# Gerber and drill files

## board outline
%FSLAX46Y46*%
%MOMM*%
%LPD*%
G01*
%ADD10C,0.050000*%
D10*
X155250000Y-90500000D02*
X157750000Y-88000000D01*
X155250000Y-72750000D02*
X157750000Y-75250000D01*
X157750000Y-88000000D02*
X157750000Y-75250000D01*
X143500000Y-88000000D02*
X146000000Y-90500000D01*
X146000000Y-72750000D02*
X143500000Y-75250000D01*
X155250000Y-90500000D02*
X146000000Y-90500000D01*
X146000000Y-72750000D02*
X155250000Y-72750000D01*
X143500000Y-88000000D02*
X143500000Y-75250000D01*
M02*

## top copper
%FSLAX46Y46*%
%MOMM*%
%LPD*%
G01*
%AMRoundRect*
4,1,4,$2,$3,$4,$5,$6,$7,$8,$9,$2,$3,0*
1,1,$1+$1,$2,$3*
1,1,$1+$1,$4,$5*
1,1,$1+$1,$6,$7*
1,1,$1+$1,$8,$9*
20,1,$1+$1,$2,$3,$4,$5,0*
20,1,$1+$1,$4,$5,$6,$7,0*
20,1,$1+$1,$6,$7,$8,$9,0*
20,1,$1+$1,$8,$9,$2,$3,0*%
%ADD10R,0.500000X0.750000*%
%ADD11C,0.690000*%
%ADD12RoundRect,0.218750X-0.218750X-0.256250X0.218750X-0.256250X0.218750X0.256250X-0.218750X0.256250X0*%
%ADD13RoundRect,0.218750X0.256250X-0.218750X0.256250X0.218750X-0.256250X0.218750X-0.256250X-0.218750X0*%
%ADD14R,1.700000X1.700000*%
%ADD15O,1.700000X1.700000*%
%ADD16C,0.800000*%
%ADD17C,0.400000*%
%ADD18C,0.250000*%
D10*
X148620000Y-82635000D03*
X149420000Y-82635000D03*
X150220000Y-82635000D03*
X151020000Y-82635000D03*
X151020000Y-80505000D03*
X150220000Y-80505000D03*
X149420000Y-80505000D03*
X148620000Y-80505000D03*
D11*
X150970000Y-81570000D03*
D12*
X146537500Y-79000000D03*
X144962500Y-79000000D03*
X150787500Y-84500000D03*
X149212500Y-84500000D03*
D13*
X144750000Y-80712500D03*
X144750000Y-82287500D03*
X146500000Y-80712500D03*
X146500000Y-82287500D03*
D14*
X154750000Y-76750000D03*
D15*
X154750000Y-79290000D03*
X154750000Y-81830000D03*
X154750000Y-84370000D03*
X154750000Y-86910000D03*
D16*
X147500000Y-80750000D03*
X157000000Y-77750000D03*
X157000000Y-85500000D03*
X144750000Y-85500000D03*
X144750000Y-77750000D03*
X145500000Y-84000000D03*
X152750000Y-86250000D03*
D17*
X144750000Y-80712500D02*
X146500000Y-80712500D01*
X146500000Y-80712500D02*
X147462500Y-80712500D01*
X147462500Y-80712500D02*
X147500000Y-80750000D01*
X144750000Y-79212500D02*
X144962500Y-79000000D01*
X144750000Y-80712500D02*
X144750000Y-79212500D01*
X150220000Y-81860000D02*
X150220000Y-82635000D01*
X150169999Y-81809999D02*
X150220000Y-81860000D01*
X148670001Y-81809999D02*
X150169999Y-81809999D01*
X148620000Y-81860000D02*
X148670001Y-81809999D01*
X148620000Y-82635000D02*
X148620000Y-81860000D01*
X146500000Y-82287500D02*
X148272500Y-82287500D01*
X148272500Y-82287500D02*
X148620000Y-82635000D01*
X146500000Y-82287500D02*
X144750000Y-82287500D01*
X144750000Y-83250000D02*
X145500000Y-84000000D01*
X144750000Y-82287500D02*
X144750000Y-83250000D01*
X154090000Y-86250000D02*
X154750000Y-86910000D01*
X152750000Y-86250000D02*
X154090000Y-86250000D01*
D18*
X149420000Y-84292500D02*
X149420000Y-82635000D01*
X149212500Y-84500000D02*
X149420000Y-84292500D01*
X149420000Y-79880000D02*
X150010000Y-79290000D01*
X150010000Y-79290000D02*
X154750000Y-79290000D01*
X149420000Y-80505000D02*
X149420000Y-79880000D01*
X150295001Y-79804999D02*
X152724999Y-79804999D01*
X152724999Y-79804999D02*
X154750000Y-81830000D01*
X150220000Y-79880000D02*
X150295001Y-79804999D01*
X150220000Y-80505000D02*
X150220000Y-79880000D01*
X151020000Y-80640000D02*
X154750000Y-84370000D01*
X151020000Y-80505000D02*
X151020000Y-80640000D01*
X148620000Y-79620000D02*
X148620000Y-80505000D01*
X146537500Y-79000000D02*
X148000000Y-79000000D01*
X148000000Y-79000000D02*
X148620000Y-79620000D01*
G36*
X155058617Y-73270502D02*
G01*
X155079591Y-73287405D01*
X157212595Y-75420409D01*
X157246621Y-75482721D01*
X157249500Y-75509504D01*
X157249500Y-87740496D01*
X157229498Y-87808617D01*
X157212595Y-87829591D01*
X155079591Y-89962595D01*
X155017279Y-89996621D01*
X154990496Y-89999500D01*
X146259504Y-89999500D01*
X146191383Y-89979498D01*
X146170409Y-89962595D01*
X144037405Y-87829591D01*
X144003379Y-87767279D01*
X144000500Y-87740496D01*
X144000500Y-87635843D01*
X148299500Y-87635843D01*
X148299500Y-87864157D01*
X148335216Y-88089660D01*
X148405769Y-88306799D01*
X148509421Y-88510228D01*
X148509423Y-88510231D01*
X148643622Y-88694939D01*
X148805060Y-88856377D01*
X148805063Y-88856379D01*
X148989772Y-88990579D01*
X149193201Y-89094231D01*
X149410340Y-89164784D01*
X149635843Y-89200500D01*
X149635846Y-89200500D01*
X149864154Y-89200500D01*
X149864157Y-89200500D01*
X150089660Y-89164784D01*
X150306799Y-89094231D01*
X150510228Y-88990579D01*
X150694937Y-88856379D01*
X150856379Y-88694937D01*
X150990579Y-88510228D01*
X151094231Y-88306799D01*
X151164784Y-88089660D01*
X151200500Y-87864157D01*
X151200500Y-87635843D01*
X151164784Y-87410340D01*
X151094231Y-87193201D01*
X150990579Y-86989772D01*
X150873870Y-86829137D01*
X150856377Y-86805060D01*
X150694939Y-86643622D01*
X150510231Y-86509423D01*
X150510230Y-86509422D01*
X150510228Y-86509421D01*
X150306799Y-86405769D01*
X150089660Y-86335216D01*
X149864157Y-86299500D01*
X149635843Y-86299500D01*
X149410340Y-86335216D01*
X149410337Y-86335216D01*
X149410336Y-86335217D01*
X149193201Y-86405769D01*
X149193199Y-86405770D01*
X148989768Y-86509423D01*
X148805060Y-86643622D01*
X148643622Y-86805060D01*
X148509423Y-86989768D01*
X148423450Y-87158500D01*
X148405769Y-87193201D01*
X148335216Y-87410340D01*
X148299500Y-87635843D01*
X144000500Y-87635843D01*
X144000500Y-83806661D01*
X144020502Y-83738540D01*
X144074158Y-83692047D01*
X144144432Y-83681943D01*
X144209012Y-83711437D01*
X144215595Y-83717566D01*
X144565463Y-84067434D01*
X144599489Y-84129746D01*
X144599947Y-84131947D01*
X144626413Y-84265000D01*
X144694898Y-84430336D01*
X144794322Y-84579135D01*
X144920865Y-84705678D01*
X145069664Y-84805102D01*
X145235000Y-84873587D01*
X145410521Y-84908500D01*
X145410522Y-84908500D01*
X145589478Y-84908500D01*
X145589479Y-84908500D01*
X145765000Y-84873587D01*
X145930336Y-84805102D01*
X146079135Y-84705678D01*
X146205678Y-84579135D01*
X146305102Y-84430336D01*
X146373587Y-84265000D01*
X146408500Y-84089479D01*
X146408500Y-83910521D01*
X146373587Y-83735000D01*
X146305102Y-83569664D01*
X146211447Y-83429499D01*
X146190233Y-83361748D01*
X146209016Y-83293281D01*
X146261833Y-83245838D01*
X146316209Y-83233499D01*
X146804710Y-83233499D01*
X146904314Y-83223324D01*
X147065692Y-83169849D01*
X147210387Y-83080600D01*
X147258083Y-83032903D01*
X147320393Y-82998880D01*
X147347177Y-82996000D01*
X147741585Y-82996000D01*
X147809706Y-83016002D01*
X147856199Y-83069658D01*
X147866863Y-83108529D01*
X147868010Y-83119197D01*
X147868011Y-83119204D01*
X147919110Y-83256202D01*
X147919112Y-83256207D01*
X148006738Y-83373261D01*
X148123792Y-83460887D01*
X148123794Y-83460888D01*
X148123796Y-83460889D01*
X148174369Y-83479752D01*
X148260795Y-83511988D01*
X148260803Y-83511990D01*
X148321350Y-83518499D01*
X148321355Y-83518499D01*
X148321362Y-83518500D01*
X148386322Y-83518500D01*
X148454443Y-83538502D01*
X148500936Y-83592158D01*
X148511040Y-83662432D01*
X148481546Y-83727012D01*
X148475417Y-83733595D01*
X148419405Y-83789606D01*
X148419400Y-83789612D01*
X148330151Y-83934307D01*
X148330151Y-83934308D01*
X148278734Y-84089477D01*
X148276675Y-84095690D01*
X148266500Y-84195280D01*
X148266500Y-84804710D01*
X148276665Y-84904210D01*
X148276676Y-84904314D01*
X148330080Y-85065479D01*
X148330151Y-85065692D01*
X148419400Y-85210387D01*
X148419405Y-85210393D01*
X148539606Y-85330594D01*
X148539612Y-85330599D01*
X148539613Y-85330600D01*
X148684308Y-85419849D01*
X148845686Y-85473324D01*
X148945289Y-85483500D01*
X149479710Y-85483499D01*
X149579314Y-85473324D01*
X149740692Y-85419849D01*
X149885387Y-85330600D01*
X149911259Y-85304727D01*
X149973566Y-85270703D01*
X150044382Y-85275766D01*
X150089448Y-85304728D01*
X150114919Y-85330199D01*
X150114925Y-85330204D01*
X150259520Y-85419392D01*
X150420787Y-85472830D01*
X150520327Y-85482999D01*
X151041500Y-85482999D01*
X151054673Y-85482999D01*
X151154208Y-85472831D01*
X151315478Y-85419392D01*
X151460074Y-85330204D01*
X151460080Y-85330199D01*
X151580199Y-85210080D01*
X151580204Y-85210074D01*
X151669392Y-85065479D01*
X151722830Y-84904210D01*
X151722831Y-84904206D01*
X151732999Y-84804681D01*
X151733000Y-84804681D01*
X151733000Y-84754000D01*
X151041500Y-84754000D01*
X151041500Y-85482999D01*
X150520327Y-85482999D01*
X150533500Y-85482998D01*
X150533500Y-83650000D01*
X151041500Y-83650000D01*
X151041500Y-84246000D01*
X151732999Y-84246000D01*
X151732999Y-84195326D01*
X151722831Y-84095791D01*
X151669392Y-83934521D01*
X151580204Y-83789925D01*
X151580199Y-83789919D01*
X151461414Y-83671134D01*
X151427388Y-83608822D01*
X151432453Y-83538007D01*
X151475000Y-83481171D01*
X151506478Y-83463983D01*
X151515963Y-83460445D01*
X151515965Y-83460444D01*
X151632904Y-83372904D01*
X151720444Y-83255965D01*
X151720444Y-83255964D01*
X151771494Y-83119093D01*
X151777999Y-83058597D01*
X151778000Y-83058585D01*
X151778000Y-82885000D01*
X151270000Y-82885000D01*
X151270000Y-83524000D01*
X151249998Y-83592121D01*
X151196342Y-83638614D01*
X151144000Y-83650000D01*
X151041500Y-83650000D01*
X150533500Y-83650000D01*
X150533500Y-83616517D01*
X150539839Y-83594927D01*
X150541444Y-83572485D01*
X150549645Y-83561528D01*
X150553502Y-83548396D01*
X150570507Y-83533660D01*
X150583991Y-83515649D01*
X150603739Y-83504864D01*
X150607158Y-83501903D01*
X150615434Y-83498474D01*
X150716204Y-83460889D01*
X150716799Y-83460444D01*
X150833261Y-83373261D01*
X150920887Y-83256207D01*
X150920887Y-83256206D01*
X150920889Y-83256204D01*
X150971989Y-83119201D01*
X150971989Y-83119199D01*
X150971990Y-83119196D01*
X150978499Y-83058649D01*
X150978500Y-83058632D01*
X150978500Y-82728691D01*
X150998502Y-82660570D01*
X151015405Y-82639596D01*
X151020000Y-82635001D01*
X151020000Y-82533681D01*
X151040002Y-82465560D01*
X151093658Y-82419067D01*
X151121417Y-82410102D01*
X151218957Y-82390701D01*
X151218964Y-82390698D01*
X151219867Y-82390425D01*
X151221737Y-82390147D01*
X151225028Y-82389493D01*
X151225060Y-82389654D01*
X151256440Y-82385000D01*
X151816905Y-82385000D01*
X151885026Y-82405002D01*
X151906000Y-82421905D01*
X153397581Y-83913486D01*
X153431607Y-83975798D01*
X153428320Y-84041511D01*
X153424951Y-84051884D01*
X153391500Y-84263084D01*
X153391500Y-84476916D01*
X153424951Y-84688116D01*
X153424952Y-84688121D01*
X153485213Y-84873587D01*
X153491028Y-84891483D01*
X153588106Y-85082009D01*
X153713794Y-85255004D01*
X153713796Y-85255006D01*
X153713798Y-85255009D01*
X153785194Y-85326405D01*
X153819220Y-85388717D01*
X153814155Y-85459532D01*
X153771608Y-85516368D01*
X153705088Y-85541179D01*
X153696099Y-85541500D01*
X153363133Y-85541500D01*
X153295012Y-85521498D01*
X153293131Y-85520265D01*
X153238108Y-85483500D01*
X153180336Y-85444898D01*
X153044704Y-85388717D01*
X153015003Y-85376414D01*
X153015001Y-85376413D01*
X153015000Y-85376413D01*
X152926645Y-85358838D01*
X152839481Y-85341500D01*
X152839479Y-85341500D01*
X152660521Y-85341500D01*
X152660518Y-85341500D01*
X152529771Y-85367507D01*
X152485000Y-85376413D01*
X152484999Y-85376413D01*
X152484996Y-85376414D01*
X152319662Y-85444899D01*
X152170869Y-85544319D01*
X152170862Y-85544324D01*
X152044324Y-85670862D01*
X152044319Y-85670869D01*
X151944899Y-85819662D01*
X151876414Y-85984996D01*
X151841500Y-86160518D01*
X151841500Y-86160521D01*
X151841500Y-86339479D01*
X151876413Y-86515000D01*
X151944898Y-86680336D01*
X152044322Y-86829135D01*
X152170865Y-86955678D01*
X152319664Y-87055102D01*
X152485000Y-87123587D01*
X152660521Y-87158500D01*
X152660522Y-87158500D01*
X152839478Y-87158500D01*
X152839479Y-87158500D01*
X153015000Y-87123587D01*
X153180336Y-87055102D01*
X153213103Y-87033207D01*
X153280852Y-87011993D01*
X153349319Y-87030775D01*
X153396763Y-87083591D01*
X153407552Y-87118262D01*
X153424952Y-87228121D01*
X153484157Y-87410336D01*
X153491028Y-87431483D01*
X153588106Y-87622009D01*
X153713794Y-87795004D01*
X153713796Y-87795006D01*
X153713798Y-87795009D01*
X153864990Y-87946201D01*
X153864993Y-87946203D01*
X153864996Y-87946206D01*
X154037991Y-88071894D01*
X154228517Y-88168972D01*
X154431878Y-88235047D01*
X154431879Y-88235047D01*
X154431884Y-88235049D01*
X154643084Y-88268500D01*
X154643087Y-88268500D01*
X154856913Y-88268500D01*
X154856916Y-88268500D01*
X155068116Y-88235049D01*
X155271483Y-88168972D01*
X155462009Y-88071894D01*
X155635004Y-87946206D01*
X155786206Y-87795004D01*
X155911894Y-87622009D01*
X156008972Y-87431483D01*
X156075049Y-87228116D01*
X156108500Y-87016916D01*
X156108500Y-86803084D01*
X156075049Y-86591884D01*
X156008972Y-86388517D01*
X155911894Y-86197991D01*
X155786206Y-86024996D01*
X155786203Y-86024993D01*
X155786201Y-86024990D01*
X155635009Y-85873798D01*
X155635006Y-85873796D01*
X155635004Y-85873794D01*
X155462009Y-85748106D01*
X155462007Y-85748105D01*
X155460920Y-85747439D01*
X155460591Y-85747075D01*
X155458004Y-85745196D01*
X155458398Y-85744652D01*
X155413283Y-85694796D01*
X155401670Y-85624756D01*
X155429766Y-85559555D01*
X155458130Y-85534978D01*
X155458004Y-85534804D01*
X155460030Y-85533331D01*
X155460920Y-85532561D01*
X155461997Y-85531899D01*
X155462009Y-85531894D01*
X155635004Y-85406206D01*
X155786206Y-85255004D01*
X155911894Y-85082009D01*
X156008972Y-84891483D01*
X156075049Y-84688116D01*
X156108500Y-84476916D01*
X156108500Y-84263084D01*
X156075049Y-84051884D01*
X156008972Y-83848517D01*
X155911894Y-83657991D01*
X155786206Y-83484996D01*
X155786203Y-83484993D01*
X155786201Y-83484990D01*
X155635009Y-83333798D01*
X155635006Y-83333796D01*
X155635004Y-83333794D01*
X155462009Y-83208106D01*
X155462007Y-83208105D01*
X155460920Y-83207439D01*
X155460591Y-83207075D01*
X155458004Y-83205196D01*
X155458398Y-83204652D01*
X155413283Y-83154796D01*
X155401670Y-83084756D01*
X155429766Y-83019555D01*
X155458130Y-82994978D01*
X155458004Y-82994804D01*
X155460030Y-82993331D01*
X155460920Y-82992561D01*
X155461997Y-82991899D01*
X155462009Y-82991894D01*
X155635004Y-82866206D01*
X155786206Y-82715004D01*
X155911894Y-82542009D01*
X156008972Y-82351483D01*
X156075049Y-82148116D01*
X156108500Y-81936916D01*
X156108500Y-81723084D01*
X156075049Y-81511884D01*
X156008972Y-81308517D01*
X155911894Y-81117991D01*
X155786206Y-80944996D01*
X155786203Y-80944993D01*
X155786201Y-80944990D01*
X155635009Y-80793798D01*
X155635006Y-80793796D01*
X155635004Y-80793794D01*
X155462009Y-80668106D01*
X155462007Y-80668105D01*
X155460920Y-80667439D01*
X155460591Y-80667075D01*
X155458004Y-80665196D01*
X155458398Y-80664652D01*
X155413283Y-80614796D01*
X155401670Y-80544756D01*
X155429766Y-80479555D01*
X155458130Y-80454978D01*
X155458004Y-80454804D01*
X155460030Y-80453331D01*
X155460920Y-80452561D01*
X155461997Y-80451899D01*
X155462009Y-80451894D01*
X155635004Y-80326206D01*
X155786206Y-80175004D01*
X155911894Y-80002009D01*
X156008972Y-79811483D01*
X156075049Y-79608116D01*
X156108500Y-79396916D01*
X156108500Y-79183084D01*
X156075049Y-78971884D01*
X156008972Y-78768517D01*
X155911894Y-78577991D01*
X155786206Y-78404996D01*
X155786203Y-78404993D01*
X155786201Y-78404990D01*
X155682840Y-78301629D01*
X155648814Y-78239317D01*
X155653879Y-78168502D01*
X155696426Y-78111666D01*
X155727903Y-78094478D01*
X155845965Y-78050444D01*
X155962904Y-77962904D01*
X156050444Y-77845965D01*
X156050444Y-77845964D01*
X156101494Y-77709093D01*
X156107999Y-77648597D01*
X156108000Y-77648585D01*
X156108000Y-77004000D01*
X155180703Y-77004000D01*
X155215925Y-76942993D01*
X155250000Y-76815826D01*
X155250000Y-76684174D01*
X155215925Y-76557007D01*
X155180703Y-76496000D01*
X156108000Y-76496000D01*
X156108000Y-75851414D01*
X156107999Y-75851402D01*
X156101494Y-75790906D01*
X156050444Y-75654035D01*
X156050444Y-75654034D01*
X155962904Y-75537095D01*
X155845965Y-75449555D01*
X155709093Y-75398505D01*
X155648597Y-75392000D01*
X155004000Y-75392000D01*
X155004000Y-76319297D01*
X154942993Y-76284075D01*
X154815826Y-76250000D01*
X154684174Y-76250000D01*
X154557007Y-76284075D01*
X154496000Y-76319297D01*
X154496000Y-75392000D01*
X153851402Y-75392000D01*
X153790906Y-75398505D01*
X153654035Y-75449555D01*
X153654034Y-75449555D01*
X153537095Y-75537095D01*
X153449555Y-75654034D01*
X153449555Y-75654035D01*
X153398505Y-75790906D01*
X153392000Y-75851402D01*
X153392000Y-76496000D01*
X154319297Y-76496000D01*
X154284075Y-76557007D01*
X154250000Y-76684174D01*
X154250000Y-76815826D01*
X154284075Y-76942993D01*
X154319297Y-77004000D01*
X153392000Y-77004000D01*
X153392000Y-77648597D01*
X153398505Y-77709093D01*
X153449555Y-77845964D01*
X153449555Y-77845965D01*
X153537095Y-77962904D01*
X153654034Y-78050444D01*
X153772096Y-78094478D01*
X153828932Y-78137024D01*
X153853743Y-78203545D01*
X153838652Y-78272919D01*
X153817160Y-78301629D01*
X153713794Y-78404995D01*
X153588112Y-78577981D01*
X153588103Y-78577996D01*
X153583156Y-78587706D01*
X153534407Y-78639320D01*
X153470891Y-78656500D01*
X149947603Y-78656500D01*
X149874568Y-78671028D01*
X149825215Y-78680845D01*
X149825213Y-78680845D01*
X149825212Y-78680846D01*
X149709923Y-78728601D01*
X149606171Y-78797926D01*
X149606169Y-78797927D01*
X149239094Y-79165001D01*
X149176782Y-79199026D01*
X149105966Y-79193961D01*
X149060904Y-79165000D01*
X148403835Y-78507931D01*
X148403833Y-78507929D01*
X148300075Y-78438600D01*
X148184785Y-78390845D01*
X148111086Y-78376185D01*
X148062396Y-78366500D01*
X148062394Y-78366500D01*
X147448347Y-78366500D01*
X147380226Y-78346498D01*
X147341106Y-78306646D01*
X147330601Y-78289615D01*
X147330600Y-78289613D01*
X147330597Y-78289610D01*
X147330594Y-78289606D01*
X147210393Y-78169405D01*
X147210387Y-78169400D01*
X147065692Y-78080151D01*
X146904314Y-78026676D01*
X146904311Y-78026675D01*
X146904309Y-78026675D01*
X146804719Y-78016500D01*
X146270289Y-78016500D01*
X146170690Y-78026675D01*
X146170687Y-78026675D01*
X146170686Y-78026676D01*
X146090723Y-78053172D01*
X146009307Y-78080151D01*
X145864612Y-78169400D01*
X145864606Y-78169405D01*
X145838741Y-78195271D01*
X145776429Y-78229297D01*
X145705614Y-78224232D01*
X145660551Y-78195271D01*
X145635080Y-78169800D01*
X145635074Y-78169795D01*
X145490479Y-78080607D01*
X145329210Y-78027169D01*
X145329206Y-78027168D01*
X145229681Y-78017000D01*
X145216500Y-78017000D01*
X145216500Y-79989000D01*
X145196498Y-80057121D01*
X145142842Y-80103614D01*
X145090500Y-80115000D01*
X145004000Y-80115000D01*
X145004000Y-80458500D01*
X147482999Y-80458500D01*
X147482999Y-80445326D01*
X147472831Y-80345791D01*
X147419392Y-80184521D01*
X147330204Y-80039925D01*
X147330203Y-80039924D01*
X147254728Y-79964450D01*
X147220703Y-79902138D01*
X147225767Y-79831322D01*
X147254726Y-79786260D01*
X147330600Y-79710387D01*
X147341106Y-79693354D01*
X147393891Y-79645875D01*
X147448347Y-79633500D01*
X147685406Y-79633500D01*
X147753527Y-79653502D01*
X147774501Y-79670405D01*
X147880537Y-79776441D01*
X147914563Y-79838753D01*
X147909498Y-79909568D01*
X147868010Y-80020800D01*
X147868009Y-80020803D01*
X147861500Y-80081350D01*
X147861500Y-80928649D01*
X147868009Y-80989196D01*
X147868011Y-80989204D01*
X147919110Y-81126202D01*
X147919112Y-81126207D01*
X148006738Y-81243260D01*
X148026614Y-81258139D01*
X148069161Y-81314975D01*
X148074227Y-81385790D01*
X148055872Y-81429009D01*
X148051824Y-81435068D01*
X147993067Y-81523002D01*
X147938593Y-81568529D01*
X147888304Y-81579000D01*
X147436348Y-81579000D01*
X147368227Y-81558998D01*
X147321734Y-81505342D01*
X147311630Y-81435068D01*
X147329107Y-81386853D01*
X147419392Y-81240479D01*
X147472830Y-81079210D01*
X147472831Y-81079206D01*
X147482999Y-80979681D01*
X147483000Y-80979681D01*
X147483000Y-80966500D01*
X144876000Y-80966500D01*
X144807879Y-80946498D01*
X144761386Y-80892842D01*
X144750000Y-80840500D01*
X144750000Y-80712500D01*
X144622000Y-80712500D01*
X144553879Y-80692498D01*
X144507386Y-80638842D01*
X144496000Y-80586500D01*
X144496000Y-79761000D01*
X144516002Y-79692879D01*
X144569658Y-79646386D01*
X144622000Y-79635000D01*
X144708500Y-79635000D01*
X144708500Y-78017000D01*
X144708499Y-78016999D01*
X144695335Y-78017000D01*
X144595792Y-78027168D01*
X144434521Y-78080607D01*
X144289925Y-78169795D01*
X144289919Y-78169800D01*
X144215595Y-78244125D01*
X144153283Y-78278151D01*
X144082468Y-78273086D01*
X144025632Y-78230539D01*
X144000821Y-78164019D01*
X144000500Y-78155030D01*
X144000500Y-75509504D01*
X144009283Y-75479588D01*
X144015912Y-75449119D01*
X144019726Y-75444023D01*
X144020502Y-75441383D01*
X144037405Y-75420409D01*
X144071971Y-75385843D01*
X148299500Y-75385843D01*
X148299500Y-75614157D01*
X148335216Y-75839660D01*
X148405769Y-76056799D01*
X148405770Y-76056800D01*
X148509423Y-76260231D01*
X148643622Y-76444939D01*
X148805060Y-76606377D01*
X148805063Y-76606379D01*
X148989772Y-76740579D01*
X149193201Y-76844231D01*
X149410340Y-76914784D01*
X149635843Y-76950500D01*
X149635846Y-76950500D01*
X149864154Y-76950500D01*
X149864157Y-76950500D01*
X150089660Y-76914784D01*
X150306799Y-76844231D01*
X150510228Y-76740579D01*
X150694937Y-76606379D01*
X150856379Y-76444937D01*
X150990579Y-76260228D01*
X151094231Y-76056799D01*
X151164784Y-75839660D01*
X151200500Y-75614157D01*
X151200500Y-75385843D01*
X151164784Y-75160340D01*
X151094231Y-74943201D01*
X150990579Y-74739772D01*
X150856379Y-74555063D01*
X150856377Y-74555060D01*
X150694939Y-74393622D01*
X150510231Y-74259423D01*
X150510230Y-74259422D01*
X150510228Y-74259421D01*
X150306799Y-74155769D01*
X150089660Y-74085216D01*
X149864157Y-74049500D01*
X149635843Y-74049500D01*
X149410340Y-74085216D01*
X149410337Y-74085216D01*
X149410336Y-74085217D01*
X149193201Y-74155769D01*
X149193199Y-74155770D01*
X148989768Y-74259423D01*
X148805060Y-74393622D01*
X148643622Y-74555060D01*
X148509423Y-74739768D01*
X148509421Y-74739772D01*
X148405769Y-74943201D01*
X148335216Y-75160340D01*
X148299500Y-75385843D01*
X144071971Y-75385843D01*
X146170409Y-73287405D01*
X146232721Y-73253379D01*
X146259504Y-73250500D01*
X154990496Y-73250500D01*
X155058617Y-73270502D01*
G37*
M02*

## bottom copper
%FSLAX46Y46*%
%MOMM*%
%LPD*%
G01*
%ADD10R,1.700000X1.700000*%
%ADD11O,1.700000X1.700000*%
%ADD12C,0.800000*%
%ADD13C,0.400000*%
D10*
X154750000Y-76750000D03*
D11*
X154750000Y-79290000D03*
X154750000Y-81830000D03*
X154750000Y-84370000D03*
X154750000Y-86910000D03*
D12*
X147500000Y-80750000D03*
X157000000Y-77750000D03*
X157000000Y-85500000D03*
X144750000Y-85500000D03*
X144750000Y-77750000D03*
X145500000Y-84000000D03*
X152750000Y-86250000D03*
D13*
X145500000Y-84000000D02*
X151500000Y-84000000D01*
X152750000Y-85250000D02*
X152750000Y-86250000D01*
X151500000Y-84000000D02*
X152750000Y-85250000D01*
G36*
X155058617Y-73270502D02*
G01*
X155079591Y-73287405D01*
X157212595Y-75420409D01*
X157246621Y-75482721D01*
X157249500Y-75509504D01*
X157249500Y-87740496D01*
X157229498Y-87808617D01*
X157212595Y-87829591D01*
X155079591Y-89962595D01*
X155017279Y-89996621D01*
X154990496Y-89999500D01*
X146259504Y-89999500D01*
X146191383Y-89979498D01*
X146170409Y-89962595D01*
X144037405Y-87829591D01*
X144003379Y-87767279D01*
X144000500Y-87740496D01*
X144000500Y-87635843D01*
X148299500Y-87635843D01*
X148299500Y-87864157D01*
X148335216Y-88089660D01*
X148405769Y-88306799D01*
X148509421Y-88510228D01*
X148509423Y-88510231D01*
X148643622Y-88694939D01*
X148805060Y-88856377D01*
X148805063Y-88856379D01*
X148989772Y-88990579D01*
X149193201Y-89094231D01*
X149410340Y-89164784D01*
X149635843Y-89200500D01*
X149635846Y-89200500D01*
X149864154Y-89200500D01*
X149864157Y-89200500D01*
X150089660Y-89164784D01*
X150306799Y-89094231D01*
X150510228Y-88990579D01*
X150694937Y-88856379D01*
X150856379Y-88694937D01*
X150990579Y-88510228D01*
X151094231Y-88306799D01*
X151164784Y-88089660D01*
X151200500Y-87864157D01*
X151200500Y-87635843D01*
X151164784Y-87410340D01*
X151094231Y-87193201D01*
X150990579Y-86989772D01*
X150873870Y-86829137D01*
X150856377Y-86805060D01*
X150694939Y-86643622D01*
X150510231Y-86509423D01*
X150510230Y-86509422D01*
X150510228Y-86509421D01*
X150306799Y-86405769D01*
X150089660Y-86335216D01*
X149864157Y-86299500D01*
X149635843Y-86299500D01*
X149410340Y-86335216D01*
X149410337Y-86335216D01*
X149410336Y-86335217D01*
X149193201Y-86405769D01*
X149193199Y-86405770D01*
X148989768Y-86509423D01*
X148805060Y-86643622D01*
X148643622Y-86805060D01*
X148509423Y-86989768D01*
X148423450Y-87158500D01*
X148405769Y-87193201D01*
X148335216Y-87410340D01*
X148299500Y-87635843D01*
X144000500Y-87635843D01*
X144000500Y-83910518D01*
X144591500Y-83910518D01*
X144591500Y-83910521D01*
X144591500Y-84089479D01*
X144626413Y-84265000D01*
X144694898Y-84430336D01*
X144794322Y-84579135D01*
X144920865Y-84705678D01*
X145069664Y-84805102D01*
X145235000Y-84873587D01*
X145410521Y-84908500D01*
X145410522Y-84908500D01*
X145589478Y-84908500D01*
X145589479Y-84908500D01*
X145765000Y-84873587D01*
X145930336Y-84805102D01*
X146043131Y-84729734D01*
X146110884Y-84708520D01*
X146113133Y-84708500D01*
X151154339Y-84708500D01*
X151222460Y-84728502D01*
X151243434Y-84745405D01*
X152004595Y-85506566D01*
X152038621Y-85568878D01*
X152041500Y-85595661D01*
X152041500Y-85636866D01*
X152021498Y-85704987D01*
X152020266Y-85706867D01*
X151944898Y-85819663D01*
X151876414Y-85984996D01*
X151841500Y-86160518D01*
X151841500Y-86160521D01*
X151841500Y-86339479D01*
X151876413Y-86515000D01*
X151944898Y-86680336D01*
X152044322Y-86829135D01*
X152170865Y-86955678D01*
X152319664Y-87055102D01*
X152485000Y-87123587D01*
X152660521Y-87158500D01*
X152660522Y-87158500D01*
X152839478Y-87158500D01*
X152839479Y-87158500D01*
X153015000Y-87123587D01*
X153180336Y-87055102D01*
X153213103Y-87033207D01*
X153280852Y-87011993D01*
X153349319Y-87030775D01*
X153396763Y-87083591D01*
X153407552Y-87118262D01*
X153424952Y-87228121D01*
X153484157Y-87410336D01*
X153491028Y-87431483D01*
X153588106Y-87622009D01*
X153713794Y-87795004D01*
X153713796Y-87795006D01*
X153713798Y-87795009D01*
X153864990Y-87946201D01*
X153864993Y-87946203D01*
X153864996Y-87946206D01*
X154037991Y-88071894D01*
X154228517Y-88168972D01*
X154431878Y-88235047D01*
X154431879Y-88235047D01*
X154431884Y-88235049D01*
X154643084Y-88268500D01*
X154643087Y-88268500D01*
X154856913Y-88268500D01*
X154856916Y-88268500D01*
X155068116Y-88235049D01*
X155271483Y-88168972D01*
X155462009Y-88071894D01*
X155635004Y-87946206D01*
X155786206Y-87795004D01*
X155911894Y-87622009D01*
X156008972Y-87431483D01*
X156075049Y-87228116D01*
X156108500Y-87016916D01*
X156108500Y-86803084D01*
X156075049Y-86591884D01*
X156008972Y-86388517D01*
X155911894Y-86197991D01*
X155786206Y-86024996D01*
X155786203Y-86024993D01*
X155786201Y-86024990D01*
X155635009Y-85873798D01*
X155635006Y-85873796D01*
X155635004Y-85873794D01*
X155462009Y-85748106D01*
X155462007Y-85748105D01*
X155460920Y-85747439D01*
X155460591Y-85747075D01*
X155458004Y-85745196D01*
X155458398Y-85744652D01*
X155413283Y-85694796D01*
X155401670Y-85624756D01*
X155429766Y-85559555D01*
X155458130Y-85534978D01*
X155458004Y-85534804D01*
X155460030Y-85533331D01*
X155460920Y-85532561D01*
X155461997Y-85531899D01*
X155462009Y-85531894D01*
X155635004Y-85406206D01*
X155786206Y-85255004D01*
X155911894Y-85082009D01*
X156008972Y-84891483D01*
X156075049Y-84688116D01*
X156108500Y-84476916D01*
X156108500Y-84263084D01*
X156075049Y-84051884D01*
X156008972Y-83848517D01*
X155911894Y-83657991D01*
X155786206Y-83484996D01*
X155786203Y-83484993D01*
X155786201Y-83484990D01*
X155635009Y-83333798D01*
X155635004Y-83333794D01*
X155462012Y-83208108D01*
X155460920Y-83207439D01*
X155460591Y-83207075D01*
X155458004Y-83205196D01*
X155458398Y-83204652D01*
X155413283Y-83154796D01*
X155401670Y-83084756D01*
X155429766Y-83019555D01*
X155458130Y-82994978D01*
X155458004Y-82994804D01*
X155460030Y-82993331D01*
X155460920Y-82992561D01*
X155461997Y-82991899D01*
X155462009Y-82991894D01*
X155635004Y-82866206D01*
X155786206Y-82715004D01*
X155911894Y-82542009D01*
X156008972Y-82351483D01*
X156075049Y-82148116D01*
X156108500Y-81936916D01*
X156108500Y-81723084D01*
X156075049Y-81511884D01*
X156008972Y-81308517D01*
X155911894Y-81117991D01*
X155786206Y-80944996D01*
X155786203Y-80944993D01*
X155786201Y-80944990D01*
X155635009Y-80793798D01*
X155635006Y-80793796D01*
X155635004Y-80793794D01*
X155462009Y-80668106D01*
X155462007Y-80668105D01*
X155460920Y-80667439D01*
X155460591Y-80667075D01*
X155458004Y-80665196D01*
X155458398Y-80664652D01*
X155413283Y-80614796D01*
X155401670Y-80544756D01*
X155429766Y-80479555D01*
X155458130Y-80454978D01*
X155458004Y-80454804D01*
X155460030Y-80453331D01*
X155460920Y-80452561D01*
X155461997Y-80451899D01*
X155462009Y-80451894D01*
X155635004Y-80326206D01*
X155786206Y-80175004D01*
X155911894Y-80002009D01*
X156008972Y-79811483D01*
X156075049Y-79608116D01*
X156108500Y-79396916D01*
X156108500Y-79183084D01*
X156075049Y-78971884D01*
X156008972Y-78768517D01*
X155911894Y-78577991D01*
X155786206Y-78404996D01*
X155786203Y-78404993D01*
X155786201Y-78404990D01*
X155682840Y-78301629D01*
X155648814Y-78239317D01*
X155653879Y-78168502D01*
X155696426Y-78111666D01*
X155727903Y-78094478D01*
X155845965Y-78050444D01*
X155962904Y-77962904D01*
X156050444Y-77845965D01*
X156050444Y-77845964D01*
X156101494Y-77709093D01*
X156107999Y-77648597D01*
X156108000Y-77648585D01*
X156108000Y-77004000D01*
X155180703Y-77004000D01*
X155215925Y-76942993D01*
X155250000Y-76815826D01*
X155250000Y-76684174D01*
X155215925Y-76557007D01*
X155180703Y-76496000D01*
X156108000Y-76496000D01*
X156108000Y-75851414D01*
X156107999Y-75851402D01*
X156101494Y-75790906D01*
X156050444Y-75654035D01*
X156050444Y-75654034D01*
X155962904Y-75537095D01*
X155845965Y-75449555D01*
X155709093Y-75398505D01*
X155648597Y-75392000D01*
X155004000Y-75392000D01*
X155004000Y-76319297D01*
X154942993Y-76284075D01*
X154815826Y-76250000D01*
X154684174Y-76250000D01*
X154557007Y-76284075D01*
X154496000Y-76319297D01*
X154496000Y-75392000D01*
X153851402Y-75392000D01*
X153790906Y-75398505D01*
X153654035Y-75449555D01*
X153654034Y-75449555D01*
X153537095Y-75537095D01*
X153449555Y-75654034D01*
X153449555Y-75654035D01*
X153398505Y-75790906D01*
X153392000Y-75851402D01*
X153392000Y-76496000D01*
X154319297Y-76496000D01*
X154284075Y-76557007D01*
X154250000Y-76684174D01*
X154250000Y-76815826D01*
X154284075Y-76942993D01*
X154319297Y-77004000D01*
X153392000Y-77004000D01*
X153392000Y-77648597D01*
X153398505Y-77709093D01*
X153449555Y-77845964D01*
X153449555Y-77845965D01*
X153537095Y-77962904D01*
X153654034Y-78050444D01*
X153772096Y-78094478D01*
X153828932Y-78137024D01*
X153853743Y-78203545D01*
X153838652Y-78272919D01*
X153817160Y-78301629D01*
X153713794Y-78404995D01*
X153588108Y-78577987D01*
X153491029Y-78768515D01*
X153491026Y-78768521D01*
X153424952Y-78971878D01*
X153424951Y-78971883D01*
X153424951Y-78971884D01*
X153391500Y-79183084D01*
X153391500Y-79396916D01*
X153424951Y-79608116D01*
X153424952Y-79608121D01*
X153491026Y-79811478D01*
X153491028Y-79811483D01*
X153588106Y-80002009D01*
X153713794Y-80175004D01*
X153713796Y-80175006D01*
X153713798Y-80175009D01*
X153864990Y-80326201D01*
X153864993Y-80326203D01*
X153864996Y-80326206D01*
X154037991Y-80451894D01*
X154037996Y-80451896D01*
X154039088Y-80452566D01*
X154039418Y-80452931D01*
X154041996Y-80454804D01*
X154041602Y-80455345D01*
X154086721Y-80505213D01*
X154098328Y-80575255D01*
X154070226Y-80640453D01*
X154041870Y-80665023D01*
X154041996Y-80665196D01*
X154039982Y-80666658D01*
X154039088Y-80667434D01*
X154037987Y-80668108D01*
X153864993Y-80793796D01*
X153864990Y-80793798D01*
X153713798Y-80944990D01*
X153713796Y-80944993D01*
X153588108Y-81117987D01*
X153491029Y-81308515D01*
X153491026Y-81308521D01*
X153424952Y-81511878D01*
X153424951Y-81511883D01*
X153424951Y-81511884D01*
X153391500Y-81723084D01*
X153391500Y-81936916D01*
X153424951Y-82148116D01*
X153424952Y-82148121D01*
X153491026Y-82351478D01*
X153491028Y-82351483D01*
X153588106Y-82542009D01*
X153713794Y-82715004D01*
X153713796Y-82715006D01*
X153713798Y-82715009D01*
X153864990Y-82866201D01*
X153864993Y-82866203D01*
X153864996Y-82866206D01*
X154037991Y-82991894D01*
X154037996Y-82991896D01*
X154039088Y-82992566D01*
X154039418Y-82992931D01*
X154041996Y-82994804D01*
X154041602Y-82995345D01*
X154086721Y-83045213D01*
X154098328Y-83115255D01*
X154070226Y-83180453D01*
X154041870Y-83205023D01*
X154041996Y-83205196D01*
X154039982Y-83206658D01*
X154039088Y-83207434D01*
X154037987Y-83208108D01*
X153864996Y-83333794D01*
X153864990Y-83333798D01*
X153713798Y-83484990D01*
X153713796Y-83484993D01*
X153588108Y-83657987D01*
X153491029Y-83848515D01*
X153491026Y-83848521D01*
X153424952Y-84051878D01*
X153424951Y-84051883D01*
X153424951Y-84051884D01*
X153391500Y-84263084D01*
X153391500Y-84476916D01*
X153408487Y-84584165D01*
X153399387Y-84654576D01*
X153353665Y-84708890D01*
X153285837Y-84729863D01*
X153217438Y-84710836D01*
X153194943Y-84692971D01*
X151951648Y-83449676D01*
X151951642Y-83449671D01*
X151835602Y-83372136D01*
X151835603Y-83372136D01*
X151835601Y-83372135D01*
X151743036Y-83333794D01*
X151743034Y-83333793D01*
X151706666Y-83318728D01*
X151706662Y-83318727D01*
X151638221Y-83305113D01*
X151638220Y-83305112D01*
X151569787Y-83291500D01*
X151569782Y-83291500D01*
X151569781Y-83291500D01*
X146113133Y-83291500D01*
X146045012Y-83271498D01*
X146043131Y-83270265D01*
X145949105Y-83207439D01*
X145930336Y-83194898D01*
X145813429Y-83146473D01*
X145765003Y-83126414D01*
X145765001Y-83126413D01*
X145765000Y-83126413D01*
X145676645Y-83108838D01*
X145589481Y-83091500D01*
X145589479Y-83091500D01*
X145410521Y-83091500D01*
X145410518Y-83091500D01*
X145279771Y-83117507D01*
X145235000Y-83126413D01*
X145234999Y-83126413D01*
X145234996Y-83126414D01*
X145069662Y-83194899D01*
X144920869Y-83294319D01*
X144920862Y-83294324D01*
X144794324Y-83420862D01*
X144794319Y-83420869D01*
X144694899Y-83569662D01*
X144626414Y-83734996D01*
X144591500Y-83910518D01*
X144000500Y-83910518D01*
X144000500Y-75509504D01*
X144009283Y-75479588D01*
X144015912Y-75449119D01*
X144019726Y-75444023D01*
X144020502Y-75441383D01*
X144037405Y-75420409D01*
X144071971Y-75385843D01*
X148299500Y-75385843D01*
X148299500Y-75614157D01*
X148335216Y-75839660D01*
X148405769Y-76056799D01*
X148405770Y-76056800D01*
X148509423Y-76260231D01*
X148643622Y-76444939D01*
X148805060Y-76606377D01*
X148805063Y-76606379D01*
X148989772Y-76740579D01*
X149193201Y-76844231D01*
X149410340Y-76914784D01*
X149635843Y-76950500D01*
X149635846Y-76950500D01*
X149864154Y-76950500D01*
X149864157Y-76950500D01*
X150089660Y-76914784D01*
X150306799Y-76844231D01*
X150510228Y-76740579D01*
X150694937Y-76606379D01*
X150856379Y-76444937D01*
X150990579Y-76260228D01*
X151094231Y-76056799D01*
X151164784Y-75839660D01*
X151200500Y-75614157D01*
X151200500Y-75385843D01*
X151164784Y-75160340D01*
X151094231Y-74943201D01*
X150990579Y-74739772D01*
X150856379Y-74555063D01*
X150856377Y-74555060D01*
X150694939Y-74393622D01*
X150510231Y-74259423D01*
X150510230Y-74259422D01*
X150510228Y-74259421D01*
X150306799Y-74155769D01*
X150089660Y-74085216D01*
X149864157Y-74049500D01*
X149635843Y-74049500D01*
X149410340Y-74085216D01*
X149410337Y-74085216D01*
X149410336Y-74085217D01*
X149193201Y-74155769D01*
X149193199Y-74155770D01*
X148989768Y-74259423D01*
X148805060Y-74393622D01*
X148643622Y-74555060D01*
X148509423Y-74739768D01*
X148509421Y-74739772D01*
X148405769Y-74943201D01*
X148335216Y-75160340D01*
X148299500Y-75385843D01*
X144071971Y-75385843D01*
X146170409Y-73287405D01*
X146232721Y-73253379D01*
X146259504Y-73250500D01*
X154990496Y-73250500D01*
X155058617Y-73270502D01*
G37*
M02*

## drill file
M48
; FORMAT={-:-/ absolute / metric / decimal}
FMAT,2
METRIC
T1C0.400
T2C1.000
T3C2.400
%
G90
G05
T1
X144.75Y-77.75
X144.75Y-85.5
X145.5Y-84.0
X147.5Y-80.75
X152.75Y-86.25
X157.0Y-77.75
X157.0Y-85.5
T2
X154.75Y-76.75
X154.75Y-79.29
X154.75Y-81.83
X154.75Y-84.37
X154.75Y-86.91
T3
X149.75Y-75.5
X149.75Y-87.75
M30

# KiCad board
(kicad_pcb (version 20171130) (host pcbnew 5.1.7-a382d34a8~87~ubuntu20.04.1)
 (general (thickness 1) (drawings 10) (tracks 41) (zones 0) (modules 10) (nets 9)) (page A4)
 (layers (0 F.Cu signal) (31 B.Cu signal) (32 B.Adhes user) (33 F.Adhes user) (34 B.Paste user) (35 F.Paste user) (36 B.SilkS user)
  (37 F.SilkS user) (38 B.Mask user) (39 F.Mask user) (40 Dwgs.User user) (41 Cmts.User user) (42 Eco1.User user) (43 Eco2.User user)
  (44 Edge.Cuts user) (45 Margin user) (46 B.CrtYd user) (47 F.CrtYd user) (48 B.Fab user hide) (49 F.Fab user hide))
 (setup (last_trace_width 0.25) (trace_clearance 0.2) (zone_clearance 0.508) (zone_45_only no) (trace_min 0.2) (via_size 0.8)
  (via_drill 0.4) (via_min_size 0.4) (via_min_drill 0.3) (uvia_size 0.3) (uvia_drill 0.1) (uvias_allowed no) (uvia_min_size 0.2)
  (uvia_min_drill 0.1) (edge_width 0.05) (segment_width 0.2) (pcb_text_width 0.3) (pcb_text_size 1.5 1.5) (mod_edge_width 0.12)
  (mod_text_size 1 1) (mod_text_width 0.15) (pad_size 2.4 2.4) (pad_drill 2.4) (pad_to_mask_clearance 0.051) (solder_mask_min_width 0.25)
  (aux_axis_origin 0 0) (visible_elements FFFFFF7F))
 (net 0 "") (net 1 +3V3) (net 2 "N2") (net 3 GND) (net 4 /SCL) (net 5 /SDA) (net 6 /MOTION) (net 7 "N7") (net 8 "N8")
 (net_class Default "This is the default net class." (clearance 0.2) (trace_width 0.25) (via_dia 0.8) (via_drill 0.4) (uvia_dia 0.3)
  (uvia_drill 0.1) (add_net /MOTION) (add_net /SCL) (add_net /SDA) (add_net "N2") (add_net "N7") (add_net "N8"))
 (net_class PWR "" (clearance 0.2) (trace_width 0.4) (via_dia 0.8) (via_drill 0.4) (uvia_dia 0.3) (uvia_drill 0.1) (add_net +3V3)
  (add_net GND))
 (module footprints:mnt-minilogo (layer F.Cu) (at 146.5 86.75 90)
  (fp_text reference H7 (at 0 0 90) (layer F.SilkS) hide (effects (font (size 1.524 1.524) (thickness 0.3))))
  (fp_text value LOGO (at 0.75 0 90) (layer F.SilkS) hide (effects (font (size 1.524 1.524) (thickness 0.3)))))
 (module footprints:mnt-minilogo (layer B.Cu) (at 146 86 270)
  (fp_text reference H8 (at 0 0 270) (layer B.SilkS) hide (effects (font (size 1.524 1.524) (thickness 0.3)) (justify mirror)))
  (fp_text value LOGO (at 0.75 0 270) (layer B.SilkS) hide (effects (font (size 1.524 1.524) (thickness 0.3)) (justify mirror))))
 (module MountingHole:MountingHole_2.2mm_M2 (layer F.Cu) (at 149.75 87.75)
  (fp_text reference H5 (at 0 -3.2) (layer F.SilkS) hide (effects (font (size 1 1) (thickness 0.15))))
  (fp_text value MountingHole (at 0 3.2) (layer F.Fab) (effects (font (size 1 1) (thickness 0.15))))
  (pad "" np_thru_hole circle (at 0 0) (size 2.4 2.4) (drill 2.4) (layers *.Cu *.Mask)))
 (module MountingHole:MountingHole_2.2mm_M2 (layer F.Cu) (at 149.75 75.5)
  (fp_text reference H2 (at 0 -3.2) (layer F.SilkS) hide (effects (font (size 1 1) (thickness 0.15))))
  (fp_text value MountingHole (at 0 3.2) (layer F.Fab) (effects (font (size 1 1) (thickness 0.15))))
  (pad "" np_thru_hole circle (at 0 0) (size 2.4 2.4) (drill 2.4) (layers *.Cu *.Mask)))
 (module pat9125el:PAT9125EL (layer F.Cu) (at 149.82 81.57)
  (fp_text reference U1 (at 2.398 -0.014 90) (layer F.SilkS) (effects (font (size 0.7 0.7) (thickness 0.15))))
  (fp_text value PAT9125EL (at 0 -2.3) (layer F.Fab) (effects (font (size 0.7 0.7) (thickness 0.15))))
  (pad 1 smd rect (at -1.2 1.065) (size 0.5 0.75) (layers F.Cu F.Paste F.Mask) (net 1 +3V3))
  (pad 2 smd rect (at -0.4 1.065) (size 0.5 0.75) (layers F.Cu F.Paste F.Mask) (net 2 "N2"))
  (pad 3 smd rect (at 0.4 1.065) (size 0.5 0.75) (layers F.Cu F.Paste F.Mask) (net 1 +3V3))
  (pad 4 smd rect (at 1.2 1.065) (size 0.5 0.75) (layers F.Cu F.Paste F.Mask) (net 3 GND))
  (pad 5 smd rect (at 1.2 -1.065) (size 0.5 0.75) (layers F.Cu F.Paste F.Mask) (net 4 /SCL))
  (pad 6 smd rect (at 0.4 -1.065) (size 0.5 0.75) (layers F.Cu F.Paste F.Mask) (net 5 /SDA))
  (pad 7 smd rect (at -0.4 -1.065) (size 0.5 0.75) (layers F.Cu F.Paste F.Mask) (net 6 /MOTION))
  (pad 8 smd rect (at -1.2 -1.065) (size 0.5 0.75) (layers F.Cu F.Paste F.Mask) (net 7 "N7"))
  (pad 9 smd circle (at 1.15 0) (size 0.69 0.69) (layers F.Cu F.Paste F.Mask) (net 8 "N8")))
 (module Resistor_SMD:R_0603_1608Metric (layer F.Cu) (at 145.75 79)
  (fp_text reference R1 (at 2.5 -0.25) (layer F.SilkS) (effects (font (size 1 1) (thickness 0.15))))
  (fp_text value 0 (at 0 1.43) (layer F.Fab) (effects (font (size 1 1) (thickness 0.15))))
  (pad 2 smd roundrect (at 0.7875 0) (size 0.875 0.95) (layers F.Cu F.Paste F.Mask) (roundrect_rratio 0.25) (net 7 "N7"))
  (pad 1 smd roundrect (at -0.7875 0) (size 0.875 0.95) (layers F.Cu F.Paste F.Mask) (roundrect_rratio 0.25) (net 3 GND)))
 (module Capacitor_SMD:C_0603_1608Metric (layer F.Cu) (at 150 84.5)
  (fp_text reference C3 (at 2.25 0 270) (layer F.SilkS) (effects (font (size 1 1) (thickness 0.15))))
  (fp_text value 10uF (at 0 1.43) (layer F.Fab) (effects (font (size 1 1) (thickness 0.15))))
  (pad 2 smd roundrect (at 0.7875 0) (size 0.875 0.95) (layers F.Cu F.Paste F.Mask) (roundrect_rratio 0.25) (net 3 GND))
  (pad 1 smd roundrect (at -0.7875 0) (size 0.875 0.95) (layers F.Cu F.Paste F.Mask) (roundrect_rratio 0.25) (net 2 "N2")))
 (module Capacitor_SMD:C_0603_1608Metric (layer F.Cu) (at 144.75 81.5 90)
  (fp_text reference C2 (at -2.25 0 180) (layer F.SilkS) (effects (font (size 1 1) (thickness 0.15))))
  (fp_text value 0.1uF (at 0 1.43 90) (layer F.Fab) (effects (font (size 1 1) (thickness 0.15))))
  (pad 2 smd roundrect (at 0.7875 0 90) (size 0.875 0.95) (layers F.Cu F.Paste F.Mask) (roundrect_rratio 0.25) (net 3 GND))
  (pad 1 smd roundrect (at -0.7875 0 90) (size 0.875 0.95) (layers F.Cu F.Paste F.Mask) (roundrect_rratio 0.25) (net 1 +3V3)))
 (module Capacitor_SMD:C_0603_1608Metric (layer F.Cu) (at 146.5 81.5 90)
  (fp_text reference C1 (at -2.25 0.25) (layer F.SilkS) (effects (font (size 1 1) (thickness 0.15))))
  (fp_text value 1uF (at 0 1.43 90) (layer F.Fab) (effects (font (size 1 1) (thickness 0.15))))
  (pad 2 smd roundrect (at 0.7875 0 90) (size 0.875 0.95) (layers F.Cu F.Paste F.Mask) (roundrect_rratio 0.25) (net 3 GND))
  (pad 1 smd roundrect (at -0.7875 0 90) (size 0.875 0.95) (layers F.Cu F.Paste F.Mask) (roundrect_rratio 0.25) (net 1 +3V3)))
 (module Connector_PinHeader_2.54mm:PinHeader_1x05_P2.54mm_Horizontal (layer F.Cu) (at 154.75 76.75)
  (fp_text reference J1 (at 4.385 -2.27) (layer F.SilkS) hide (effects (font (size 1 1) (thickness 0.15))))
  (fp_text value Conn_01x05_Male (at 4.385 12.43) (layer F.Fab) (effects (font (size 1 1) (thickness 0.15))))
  (pad 1 thru_hole rect (at 0 0) (size 1.7 1.7) (drill 1) (layers *.Cu *.Mask) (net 3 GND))
  (pad 2 thru_hole oval (at 0 2.54) (size 1.7 1.7) (drill 1) (layers *.Cu *.Mask) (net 6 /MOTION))
  (pad 3 thru_hole oval (at 0 5.08) (size 1.7 1.7) (drill 1) (layers *.Cu *.Mask) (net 5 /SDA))
  (pad 4 thru_hole oval (at 0 7.62) (size 1.7 1.7) (drill 1) (layers *.Cu *.Mask) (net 4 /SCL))
  (pad 5 thru_hole oval (at 0 10.16) (size 1.7 1.7) (drill 1) (layers *.Cu *.Mask) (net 1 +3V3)))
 (gr_line (start 155.25 90.5) (end 157.75 88) (layer Edge.Cuts) (width 0.05))
 (gr_line (start 155.25 72.75) (end 157.75 75.25) (layer Edge.Cuts) (width 0.05))
 (gr_line (start 157.75 88) (end 157.75 75.25) (layer Edge.Cuts) (width 0.05))
 (gr_line (start 143.5 88) (end 146 90.5) (layer Edge.Cuts) (width 0.05))
 (gr_line (start 146 72.75) (end 143.5 75.25) (layer Edge.Cuts) (width 0.05))
 (gr_line (start 155.25 90.5) (end 146 90.5) (layer Edge.Cuts) (width 0.05))
 (gr_line (start 146 72.75) (end 155.25 72.75) (layer Edge.Cuts) (width 0.05))
 (gr_line (start 143.5 88) (end 143.5 75.25) (layer Edge.Cuts) (width 0.05))
 (segment (start 144.75 80.7125) (end 146.5 80.7125) (width 0.4) (layer F.Cu) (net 3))
 (segment (start 146.5 80.7125) (end 147.4625 80.7125) (width 0.4) (layer F.Cu) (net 3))
 (via (at 147.5 80.75) (size 0.8) (drill 0.4) (layers F.Cu B.Cu) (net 3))
 (segment (start 147.4625 80.7125) (end 147.5 80.75) (width 0.4) (layer F.Cu) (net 3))
 (segment (start 144.75 79.2125) (end 144.9625 79) (width 0.4) (layer F.Cu) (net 3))
 (segment (start 144.75 80.7125) (end 144.75 79.2125) (width 0.4) (layer F.Cu) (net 3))
 (via (at 157 77.75) (size 0.8) (drill 0.4) (layers F.Cu B.Cu) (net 3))
 (via (at 157 85.5) (size 0.8) (drill 0.4) (layers F.Cu B.Cu) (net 3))
 (via (at 144.75 85.5) (size 0.8) (drill 0.4) (layers F.Cu B.Cu) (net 3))
 (via (at 144.75 77.75) (size 0.8) (drill 0.4) (layers F.Cu B.Cu) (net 3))
 (segment (start 150.22 81.86) (end 150.22 82.635) (width 0.4) (layer F.Cu) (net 1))
 (segment (start 150.169999 81.809999) (end 150.22 81.86) (width 0.4) (layer F.Cu) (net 1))
 (segment (start 148.670001 81.809999) (end 150.169999 81.809999) (width 0.4) (layer F.Cu) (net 1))
 (segment (start 148.62 81.86) (end 148.670001 81.809999) (width 0.4) (layer F.Cu) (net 1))
 (segment (start 148.62 82.635) (end 148.62 81.86) (width 0.4) (layer F.Cu) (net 1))
 (segment (start 146.5 82.2875) (end 148.2725 82.2875) (width 0.4) (layer F.Cu) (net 1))
 (segment (start 148.2725 82.2875) (end 148.62 82.635) (width 0.4) (layer F.Cu) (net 1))
 (segment (start 146.5 82.2875) (end 144.75 82.2875) (width 0.4) (layer F.Cu) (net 1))
 (via (at 145.5 84) (size 0.8) (drill 0.4) (layers F.Cu B.Cu) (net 1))
 (segment (start 144.75 83.25) (end 145.5 84) (width 0.4) (layer F.Cu) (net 1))
 (segment (start 144.75 82.2875) (end 144.75 83.25) (width 0.4) (layer F.Cu) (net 1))
 (segment (start 145.5 84) (end 151.5 84) (width 0.4) (layer B.Cu) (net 1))
 (via (at 152.75 86.25) (size 0.8) (drill 0.4) (layers F.Cu B.Cu) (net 1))
 (segment (start 152.75 85.25) (end 152.75 86.25) (width 0.4) (layer B.Cu) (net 1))
 (segment (start 151.5 84) (end 152.75 85.25) (width 0.4) (layer B.Cu) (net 1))
 (segment (start 154.09 86.25) (end 154.75 86.91) (width 0.4) (layer F.Cu) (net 1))
 (segment (start 152.75 86.25) (end 154.09 86.25) (width 0.4) (layer F.Cu) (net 1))
 (segment (start 149.42 84.2925) (end 149.42 82.635) (width 0.25) (layer F.Cu) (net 2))
 (segment (start 149.2125 84.5) (end 149.42 84.2925) (width 0.25) (layer F.Cu) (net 2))
 (segment (start 149.42 79.88) (end 150.01 79.29) (width 0.25) (layer F.Cu) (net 6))
 (segment (start 150.01 79.29) (end 154.75 79.29) (width 0.25) (layer F.Cu) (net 6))
 (segment (start 149.42 80.505) (end 149.42 79.88) (width 0.25) (layer F.Cu) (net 6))
 (segment (start 150.295001 79.804999) (end 152.724999 79.804999) (width 0.25) (layer F.Cu) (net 5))
 (segment (start 152.724999 79.804999) (end 154.75 81.83) (width 0.25) (layer F.Cu) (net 5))
 (segment (start 150.22 79.88) (end 150.295001 79.804999) (width 0.25) (layer F.Cu) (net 5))
 (segment (start 150.22 80.505) (end 150.22 79.88) (width 0.25) (layer F.Cu) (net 5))
 (segment (start 151.02 80.64) (end 154.75 84.37) (width 0.25) (layer F.Cu) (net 4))
 (segment (start 151.02 80.505) (end 151.02 80.64) (width 0.25) (layer F.Cu) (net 4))
 (segment (start 148.62 79.62) (end 148.62 80.505) (width 0.25) (layer F.Cu) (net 7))
 (segment (start 146.5375 79) (end 148 79) (width 0.25) (layer F.Cu) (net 7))
 (segment (start 148 79) (end 148.62 79.62) (width 0.25) (layer F.Cu) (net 7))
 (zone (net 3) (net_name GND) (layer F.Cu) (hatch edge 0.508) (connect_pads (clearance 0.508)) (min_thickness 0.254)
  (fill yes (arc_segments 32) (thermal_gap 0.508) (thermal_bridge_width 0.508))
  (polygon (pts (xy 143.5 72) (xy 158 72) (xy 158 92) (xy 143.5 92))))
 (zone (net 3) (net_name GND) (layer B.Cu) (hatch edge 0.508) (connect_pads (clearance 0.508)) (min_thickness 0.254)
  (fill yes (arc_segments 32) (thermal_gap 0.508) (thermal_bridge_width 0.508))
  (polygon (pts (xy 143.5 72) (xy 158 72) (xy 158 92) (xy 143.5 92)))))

